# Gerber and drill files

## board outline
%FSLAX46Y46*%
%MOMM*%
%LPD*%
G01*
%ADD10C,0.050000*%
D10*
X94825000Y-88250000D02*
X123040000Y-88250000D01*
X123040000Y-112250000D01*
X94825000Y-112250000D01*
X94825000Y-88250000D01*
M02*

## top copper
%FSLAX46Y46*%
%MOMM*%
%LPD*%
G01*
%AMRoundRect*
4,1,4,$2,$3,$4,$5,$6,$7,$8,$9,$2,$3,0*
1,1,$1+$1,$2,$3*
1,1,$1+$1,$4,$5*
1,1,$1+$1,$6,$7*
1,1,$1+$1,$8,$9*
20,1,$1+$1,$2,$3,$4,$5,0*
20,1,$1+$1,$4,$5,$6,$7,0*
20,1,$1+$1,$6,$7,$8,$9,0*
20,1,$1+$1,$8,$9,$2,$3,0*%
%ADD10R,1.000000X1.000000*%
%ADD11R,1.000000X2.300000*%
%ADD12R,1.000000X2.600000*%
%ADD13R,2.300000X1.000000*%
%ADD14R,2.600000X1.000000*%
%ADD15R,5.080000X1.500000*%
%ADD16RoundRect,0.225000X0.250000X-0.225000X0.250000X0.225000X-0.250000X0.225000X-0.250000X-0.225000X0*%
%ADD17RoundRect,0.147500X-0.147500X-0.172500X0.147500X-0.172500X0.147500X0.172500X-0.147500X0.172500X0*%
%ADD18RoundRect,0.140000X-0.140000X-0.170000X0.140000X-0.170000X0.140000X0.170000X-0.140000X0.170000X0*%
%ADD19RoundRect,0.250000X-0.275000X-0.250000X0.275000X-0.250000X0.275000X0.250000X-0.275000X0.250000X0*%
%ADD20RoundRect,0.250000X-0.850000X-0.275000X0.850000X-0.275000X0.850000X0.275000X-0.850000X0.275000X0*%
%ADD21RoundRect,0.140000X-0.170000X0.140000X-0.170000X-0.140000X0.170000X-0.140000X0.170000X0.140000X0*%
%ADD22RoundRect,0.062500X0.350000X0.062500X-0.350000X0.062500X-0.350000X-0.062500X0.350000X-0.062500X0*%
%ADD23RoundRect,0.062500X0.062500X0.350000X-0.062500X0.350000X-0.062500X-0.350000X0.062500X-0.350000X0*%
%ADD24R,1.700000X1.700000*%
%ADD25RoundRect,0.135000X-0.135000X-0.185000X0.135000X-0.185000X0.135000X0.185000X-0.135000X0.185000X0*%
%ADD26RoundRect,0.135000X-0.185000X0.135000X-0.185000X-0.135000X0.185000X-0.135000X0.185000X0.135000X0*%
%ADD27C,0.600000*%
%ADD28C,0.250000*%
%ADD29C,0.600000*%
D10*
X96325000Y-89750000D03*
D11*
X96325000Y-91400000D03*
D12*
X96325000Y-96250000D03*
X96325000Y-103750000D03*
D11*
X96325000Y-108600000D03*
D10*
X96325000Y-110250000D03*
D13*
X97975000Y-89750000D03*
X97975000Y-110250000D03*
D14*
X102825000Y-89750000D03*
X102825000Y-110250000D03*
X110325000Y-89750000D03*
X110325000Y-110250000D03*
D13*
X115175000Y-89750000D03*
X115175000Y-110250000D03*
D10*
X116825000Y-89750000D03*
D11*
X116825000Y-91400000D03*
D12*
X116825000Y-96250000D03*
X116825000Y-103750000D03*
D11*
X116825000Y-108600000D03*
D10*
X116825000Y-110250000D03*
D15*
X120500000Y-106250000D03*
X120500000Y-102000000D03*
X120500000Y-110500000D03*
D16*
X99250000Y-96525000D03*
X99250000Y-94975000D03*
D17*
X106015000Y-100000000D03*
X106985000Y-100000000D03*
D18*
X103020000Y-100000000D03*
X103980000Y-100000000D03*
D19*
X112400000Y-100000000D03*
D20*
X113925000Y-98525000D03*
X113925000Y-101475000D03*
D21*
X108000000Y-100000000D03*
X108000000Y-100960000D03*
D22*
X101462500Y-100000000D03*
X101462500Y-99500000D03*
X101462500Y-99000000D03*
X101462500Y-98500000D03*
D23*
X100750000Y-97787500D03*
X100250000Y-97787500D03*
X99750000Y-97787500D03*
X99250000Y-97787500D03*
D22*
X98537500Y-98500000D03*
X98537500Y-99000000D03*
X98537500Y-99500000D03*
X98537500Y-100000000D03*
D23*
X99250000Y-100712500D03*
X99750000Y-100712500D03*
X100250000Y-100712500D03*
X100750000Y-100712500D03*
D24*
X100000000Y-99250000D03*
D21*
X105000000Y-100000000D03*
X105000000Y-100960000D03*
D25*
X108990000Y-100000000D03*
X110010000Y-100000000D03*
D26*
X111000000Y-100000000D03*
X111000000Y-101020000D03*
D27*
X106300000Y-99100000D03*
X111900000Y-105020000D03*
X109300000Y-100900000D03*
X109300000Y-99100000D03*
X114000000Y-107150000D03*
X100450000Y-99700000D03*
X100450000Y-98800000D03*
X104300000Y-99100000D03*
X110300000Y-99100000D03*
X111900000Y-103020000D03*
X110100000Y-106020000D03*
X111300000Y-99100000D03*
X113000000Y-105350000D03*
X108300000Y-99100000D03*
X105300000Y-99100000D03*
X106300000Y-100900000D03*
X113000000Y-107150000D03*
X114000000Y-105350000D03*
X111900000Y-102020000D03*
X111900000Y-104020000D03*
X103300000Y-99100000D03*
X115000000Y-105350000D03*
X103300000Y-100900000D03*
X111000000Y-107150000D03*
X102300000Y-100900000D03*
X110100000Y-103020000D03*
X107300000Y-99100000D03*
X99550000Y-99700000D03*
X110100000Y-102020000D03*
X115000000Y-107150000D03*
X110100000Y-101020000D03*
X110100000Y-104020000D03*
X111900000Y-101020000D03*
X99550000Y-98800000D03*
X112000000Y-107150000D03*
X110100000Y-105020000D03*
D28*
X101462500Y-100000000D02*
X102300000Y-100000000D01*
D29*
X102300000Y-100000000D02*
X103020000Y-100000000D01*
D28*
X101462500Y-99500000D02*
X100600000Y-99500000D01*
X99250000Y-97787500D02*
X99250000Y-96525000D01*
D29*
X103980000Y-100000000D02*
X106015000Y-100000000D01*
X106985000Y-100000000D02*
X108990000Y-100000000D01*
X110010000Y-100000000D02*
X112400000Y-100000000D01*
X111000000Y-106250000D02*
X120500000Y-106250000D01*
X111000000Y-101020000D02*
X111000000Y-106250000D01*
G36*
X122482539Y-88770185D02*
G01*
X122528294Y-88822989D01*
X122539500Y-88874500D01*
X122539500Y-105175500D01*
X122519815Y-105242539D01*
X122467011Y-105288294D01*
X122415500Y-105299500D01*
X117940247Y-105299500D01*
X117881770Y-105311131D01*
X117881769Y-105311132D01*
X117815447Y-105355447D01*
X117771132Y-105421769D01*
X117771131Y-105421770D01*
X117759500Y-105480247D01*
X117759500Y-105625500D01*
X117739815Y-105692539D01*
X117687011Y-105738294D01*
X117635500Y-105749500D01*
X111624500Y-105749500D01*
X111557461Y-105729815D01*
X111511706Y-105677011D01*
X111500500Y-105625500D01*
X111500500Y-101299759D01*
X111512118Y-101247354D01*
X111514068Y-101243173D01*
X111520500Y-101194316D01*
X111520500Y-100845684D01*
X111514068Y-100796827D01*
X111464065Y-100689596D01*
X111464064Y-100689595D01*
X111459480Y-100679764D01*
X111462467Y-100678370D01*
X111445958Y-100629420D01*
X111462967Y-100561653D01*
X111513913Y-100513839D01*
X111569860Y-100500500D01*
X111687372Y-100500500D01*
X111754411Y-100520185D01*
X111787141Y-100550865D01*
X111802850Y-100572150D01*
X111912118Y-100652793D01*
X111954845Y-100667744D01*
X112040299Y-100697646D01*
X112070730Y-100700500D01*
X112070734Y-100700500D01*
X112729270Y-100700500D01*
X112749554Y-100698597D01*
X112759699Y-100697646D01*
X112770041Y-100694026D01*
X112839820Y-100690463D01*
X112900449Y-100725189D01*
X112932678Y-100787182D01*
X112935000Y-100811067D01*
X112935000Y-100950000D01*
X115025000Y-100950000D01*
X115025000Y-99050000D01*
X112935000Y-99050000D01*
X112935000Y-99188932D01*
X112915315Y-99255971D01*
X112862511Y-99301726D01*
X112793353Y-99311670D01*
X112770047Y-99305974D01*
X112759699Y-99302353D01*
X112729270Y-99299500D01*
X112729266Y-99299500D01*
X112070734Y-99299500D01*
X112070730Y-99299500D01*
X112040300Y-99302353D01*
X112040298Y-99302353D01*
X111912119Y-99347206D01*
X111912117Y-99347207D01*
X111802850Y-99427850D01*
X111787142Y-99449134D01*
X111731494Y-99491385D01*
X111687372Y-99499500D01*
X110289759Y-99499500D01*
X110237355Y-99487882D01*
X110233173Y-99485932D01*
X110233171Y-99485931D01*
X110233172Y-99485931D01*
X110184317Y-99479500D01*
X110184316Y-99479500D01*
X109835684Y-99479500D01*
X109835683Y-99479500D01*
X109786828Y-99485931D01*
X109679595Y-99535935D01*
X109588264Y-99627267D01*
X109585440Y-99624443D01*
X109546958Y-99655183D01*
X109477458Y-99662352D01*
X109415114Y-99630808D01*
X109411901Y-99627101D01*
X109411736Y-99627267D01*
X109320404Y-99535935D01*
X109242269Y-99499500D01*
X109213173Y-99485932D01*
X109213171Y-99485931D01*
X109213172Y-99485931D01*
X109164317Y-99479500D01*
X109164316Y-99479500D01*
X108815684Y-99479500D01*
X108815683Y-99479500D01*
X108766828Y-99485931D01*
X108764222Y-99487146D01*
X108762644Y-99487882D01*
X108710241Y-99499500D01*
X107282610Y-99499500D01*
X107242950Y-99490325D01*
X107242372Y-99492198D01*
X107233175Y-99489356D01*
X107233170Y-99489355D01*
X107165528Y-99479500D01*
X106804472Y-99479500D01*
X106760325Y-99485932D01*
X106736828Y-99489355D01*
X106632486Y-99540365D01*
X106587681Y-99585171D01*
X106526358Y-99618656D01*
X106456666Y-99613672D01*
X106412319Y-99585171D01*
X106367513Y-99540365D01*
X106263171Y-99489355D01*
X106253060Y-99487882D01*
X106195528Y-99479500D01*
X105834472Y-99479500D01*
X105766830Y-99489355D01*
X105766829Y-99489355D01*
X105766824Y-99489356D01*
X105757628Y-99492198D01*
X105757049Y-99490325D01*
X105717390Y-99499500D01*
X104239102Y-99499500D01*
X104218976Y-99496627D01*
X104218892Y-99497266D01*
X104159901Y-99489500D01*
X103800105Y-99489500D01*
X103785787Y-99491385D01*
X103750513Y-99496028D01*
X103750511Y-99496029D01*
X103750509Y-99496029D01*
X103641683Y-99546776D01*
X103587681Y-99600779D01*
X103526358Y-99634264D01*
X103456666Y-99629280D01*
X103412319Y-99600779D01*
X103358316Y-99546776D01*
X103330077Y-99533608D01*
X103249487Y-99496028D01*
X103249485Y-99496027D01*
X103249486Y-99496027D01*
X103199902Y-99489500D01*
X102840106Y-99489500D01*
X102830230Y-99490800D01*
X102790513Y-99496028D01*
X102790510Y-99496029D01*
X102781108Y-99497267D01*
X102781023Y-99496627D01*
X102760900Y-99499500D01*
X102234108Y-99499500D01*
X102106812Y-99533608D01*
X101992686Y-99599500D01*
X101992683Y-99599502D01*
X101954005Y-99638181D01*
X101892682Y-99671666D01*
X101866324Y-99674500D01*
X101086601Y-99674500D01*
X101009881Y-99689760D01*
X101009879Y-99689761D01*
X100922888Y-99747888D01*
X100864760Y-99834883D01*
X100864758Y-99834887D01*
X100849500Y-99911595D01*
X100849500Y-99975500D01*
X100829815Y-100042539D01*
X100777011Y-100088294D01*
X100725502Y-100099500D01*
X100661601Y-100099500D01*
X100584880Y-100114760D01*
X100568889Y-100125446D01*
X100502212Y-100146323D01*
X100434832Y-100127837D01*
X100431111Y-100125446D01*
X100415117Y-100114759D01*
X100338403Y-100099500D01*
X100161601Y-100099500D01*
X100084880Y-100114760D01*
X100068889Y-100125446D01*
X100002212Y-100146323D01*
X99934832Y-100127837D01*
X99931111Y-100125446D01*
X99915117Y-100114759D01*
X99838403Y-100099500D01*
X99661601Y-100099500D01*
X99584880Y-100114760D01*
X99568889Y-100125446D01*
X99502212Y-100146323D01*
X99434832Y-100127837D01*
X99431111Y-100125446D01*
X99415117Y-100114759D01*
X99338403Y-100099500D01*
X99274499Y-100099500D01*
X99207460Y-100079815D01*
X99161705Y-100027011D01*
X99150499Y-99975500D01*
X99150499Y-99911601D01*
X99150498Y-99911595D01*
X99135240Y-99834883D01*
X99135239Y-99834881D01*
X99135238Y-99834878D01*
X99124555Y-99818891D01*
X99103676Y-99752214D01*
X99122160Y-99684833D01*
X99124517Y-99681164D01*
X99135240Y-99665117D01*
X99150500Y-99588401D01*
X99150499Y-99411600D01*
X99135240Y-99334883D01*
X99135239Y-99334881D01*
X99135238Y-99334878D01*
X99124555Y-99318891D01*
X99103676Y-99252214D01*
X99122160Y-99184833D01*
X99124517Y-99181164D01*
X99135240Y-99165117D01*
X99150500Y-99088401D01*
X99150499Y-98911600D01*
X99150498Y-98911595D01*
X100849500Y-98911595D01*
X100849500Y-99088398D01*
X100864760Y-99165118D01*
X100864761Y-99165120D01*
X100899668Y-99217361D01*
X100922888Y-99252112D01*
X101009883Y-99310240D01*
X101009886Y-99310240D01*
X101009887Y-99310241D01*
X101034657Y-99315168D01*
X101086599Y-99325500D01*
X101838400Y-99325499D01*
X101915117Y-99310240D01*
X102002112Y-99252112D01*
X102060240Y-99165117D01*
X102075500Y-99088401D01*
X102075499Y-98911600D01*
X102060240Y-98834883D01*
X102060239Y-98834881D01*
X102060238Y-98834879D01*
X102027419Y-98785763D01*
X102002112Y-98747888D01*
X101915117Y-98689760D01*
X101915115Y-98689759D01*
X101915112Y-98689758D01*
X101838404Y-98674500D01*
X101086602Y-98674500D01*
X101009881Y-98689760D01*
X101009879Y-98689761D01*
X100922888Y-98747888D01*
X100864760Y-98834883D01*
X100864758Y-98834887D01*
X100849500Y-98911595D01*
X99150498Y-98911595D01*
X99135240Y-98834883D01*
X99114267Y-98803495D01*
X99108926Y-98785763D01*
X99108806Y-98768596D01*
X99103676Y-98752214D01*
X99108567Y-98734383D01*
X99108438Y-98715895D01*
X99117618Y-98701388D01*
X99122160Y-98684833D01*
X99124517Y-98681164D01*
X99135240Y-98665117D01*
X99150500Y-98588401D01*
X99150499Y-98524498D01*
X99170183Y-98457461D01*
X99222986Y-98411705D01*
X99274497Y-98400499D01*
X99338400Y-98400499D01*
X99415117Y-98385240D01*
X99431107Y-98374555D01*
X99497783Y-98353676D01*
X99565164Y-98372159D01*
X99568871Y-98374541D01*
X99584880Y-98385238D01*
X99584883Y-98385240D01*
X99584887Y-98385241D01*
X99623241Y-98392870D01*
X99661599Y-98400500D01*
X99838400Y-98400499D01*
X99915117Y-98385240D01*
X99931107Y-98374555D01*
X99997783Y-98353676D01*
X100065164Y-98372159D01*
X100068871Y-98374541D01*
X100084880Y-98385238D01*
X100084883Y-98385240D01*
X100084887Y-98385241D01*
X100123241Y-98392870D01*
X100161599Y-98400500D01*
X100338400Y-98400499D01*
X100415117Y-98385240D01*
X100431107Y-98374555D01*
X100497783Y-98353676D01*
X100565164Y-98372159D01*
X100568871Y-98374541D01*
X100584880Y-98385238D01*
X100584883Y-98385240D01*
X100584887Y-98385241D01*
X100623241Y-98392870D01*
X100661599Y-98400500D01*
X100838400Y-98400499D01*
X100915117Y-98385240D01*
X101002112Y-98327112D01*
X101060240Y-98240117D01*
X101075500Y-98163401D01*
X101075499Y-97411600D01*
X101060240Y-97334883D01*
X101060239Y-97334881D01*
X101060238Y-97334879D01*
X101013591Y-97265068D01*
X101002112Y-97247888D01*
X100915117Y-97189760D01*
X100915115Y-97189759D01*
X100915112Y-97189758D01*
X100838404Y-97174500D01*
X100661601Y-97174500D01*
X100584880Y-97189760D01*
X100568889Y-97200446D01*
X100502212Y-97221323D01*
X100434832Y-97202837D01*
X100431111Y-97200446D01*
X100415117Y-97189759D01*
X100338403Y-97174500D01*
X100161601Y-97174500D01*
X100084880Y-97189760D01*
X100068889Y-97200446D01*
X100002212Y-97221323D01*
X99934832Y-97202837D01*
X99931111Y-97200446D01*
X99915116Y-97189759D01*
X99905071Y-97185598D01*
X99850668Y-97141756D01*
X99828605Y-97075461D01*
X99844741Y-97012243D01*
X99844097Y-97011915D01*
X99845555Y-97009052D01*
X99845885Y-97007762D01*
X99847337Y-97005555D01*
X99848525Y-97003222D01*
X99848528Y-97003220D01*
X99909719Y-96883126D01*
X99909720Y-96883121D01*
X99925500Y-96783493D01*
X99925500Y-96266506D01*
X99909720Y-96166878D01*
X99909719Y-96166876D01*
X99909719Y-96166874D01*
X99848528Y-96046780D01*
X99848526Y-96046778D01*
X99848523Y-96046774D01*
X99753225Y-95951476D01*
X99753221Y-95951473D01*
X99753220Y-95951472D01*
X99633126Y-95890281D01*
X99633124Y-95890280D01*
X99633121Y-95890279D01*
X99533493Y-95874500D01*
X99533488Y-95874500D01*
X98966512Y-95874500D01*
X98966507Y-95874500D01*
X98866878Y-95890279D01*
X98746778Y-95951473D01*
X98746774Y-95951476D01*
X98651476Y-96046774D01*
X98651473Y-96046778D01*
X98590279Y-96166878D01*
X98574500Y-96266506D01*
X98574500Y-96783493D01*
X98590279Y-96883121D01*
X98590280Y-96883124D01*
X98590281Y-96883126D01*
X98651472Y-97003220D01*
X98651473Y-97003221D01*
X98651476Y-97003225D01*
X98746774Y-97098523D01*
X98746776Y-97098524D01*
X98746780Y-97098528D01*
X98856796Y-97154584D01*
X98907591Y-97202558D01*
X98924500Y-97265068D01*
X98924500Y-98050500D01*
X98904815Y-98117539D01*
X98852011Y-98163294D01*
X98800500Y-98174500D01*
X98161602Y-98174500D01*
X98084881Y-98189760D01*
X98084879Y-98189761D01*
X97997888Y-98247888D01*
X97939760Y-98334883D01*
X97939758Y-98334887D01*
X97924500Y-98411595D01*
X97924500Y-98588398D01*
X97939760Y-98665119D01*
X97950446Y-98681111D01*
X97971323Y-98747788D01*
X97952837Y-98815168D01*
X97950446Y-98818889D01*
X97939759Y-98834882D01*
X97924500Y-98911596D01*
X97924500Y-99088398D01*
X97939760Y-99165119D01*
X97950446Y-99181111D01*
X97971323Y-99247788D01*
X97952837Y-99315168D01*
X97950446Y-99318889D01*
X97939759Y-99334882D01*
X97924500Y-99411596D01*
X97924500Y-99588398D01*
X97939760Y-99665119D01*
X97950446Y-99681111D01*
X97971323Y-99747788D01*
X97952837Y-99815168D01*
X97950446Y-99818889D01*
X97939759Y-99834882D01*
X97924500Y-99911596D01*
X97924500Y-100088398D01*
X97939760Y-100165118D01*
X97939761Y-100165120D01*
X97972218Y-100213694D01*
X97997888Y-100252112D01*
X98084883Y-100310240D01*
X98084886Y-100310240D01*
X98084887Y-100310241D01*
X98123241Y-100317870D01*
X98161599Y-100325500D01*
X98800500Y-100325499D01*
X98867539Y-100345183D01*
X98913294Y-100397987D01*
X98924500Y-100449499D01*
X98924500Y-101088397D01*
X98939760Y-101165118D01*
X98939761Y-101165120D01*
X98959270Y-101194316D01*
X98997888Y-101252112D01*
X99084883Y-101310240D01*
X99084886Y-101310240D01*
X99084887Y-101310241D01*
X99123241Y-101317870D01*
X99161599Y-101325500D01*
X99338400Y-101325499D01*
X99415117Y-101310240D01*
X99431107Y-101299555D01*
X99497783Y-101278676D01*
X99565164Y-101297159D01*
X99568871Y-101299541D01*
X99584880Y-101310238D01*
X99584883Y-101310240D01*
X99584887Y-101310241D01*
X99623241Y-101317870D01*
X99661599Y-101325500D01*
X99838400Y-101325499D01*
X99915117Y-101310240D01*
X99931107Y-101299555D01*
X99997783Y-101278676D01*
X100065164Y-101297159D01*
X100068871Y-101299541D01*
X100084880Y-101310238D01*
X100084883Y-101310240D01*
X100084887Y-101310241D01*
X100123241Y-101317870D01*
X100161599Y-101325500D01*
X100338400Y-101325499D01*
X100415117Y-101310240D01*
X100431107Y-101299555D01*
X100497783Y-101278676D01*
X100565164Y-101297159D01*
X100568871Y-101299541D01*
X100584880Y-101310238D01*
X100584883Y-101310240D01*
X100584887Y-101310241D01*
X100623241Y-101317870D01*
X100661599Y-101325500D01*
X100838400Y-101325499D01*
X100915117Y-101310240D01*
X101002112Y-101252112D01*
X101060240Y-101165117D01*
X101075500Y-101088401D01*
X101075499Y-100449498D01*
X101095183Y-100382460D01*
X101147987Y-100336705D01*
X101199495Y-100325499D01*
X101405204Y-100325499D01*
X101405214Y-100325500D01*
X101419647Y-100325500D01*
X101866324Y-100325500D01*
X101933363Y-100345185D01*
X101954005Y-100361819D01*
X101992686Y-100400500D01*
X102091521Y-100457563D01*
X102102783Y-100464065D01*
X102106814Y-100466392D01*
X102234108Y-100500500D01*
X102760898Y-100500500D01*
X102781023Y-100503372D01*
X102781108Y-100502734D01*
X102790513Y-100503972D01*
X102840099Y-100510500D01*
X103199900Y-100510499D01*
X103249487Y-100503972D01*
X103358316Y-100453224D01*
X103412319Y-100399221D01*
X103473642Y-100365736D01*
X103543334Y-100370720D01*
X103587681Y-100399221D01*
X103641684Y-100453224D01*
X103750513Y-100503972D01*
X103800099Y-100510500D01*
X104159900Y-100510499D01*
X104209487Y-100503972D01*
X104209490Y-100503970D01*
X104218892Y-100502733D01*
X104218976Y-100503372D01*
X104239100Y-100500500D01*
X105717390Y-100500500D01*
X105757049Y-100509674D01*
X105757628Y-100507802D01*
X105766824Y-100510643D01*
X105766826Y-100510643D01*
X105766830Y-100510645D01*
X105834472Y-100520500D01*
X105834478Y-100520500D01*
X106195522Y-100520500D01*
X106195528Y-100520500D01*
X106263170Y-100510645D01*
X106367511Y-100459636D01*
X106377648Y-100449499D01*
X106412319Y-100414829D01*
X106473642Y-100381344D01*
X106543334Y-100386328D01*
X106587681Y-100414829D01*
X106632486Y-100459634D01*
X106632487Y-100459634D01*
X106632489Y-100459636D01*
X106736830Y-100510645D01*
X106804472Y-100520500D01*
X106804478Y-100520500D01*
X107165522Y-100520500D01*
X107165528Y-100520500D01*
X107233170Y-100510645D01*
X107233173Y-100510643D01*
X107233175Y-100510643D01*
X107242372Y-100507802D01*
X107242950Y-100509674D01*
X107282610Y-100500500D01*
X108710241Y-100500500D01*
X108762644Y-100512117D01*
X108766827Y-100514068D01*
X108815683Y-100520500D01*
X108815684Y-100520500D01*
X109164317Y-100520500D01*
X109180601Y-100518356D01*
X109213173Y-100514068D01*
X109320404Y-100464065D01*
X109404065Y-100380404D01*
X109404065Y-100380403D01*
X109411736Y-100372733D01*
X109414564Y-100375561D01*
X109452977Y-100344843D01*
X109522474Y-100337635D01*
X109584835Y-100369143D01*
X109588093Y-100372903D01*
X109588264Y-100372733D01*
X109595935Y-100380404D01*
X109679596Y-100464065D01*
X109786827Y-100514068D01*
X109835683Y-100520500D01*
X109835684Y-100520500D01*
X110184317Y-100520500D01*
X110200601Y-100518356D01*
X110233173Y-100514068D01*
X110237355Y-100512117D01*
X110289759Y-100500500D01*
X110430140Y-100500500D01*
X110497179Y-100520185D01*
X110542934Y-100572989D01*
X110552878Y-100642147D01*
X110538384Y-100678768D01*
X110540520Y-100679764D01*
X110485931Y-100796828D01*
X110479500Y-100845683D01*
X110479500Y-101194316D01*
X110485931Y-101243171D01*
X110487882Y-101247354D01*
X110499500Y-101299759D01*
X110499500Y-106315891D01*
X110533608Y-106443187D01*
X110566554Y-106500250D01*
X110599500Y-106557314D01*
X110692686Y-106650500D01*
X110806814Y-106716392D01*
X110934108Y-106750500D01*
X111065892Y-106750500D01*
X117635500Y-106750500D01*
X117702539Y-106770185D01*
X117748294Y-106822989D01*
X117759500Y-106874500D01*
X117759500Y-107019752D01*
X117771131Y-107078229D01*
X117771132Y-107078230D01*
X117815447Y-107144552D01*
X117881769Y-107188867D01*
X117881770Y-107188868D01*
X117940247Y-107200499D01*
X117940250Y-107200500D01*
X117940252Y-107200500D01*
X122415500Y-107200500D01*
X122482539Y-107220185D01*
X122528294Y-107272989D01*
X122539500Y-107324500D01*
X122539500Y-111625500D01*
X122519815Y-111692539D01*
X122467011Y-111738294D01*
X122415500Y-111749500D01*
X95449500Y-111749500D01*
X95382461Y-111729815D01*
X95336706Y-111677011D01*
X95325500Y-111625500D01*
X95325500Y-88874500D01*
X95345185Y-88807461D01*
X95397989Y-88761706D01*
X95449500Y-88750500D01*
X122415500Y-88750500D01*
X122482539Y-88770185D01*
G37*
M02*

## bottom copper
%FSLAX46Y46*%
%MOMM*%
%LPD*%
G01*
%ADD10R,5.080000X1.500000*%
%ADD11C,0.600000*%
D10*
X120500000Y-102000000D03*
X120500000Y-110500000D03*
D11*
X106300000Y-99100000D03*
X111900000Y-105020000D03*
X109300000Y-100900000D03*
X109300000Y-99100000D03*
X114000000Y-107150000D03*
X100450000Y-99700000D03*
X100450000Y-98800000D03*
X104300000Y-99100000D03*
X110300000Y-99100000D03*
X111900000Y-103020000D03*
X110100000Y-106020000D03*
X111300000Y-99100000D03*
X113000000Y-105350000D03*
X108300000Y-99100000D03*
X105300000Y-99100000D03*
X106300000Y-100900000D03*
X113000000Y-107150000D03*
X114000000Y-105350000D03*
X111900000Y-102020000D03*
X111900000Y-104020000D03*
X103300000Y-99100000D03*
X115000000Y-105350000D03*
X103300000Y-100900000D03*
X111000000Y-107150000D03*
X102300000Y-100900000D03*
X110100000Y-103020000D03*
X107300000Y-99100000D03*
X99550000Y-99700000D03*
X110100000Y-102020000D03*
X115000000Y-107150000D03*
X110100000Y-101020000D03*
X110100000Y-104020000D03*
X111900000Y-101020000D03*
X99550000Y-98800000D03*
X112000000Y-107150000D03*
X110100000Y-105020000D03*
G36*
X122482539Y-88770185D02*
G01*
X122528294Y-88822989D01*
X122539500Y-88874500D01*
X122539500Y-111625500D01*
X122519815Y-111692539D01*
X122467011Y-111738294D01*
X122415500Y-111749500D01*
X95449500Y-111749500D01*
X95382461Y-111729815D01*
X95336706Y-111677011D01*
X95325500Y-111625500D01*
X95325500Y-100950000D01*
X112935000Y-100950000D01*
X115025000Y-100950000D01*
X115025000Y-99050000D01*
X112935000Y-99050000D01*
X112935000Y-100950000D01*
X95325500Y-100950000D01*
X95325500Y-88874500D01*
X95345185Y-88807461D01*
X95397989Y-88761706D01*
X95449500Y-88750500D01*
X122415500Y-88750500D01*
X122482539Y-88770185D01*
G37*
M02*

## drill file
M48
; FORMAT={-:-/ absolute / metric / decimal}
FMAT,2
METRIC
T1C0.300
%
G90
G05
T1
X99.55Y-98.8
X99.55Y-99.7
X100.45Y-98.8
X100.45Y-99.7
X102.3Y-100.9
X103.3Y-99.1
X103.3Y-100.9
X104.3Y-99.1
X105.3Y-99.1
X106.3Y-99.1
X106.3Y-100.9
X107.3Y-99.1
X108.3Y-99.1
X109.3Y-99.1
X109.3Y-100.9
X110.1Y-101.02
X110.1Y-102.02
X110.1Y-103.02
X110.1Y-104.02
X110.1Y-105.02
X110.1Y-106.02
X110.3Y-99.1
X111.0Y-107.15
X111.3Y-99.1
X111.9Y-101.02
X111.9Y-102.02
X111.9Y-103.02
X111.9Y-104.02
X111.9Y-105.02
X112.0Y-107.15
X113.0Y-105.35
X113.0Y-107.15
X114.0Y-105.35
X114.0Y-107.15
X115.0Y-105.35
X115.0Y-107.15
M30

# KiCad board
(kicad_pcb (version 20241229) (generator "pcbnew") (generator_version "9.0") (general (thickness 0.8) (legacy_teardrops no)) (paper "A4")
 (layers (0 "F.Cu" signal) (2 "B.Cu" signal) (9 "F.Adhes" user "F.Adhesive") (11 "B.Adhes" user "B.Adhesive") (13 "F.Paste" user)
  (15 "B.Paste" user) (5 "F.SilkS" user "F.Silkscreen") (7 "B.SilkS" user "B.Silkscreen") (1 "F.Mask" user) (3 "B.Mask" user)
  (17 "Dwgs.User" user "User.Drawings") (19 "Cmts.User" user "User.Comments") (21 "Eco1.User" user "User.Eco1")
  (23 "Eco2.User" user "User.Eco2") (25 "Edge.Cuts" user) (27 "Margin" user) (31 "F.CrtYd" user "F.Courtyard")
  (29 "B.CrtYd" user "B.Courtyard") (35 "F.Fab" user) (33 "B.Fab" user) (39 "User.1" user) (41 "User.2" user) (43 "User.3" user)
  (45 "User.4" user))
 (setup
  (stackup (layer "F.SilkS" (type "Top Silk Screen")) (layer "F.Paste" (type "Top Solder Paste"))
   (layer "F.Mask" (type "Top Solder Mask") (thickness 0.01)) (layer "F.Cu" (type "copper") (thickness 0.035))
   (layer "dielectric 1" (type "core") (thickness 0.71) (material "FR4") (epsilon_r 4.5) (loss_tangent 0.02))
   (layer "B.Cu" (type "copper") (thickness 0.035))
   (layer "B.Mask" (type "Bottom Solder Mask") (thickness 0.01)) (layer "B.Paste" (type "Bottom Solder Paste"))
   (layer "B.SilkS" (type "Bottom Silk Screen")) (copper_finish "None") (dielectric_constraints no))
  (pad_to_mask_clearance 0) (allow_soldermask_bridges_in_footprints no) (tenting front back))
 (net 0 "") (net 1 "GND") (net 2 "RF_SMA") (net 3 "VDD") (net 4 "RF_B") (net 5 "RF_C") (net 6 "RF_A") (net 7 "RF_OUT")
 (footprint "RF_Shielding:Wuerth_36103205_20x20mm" (layer "F.Cu") (at 106.575 100)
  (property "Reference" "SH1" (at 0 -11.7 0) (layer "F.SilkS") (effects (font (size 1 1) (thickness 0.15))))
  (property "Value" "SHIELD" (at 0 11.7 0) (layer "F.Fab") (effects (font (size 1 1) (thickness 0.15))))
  (pad "1" smd rect (at -10.25 -10.25) (size 1 1) (layers "F.Cu" "F.Mask" "F.Paste") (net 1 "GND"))
  (pad "1" smd rect (at -10.25 -8.6) (size 1 2.3) (layers "F.Cu" "F.Mask" "F.Paste") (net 1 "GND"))
  (pad "1" smd rect (at -10.25 -3.75) (size 1 2.6) (layers "F.Cu" "F.Mask" "F.Paste") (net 1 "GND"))
  (pad "1" smd rect (at -10.25 3.75) (size 1 2.6) (layers "F.Cu" "F.Mask" "F.Paste") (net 1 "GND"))
  (pad "1" smd rect (at -10.25 8.6) (size 1 2.3) (layers "F.Cu" "F.Mask" "F.Paste") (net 1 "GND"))
  (pad "1" smd rect (at -10.25 10.25) (size 1 1) (layers "F.Cu" "F.Mask" "F.Paste") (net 1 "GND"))
  (pad "1" smd rect (at -8.6 -10.25) (size 2.3 1) (layers "F.Cu" "F.Mask" "F.Paste") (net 1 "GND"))
  (pad "1" smd rect (at -8.6 10.25) (size 2.3 1) (layers "F.Cu" "F.Mask" "F.Paste") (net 1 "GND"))
  (pad "1" smd rect (at -3.75 -10.25) (size 2.6 1) (layers "F.Cu" "F.Mask" "F.Paste") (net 1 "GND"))
  (pad "1" smd rect (at -3.75 10.25) (size 2.6 1) (layers "F.Cu" "F.Mask" "F.Paste") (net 1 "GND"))
  (pad "1" smd rect (at 3.75 -10.25) (size 2.6 1) (layers "F.Cu" "F.Mask" "F.Paste") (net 1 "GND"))
  (pad "1" smd rect (at 3.75 10.25) (size 2.6 1) (layers "F.Cu" "F.Mask" "F.Paste") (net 1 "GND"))
  (pad "1" smd rect (at 8.6 -10.25) (size 2.3 1) (layers "F.Cu" "F.Mask" "F.Paste") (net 1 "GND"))
  (pad "1" smd rect (at 8.6 10.25) (size 2.3 1) (layers "F.Cu" "F.Mask" "F.Paste") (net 1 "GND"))
  (pad "1" smd rect (at 10.25 -10.25) (size 1 1) (layers "F.Cu" "F.Mask" "F.Paste") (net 1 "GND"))
  (pad "1" smd rect (at 10.25 -8.6) (size 1 2.3) (layers "F.Cu" "F.Mask" "F.Paste") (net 1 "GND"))
  (pad "1" smd rect (at 10.25 -3.75) (size 1 2.6) (layers "F.Cu" "F.Mask" "F.Paste") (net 1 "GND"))
  (pad "1" smd rect (at 10.25 3.75) (size 1 2.6) (layers "F.Cu" "F.Mask" "F.Paste") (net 1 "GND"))
  (pad "1" smd rect (at 10.25 8.6) (size 1 2.3) (layers "F.Cu" "F.Mask" "F.Paste") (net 1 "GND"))
  (pad "1" smd rect (at 10.25 10.25) (size 1 1) (layers "F.Cu" "F.Mask" "F.Paste") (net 1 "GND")))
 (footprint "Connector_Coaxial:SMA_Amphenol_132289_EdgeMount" (layer "F.Cu") (at 120.5 106.25)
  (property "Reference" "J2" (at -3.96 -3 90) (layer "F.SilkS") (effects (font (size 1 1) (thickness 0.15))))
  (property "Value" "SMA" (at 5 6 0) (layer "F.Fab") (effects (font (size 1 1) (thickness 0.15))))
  (pad "1" smd rect (at 0 0 90) (size 1.5 5.08) (layers "F.Cu" "F.Mask" "F.Paste") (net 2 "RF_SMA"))
  (pad "2" smd rect (at 0 -4.25 90) (size 1.5 5.08) (layers "F.Cu" "F.Mask" "F.Paste") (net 1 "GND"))
  (pad "2" smd rect (at 0 -4.25 90) (size 1.5 5.08) (layers "B.Cu" "B.Mask" "B.Paste") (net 1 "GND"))
  (pad "2" smd rect (at 0 4.25 90) (size 1.5 5.08) (layers "F.Cu" "F.Mask" "F.Paste") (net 1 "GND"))
  (pad "2" smd rect (at 0 4.25 90) (size 1.5 5.08) (layers "B.Cu" "B.Mask" "B.Paste") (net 1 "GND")))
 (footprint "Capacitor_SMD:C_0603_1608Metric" (layer "F.Cu") (at 99.25 95.75 90)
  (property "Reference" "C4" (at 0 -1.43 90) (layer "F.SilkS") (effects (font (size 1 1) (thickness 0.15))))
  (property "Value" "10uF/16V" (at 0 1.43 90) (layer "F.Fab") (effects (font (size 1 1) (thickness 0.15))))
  (pad "1" smd roundrect (at -0.775 0 90) (size 0.9 0.95) (layers "F.Cu" "F.Mask" "F.Paste") (roundrect_rratio 0.25) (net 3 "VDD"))
  (pad "2" smd roundrect (at 0.775 0 90) (size 0.9 0.95) (layers "F.Cu" "F.Mask" "F.Paste") (roundrect_rratio 0.25) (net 1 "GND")))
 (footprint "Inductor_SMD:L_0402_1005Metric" (layer "F.Cu") (at 106.5 100)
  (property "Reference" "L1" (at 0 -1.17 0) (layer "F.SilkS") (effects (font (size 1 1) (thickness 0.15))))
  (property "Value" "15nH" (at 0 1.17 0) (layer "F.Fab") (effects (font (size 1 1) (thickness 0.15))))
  (pad "1" smd roundrect (at -0.485 0) (size 0.59 0.64) (layers "F.Cu" "F.Mask" "F.Paste") (roundrect_rratio 0.25) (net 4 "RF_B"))
  (pad "2" smd roundrect (at 0.485 0) (size 0.59 0.64) (layers "F.Cu" "F.Mask" "F.Paste") (roundrect_rratio 0.25) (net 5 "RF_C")))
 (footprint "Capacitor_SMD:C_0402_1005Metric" (layer "F.Cu") (at 103.5 100)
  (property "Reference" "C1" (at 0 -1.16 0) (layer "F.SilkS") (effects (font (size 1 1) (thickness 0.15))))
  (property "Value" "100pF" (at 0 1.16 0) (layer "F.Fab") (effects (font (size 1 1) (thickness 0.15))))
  (pad "1" smd roundrect (at -0.48 0) (size 0.56 0.62) (layers "F.Cu" "F.Mask" "F.Paste") (roundrect_rratio 0.25) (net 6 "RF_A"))
  (pad "2" smd roundrect (at 0.48 0) (size 0.56 0.62) (layers "F.Cu" "F.Mask" "F.Paste") (roundrect_rratio 0.25) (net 4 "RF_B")))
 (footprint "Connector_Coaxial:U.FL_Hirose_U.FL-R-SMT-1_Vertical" (layer "F.Cu") (at 113.45 100)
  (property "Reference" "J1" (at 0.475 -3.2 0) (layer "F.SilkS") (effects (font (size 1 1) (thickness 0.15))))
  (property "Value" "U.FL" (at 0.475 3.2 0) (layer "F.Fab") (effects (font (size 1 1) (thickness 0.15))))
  (pad "1" smd roundrect (at -1.05 0) (size 1.05 1) (layers "F.Cu" "F.Mask" "F.Paste") (roundrect_rratio 0.25) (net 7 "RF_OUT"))
  (pad "2" smd roundrect (at 0.475 -1.475) (size 2.2 1.05) (layers "F.Cu" "F.Mask" "F.Paste") (roundrect_rratio 0.2380952381) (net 1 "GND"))
  (pad "2" smd roundrect (at 0.475 1.475) (size 2.2 1.05) (layers "F.Cu" "F.Mask" "F.Paste") (roundrect_rratio 0.2380952381) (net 1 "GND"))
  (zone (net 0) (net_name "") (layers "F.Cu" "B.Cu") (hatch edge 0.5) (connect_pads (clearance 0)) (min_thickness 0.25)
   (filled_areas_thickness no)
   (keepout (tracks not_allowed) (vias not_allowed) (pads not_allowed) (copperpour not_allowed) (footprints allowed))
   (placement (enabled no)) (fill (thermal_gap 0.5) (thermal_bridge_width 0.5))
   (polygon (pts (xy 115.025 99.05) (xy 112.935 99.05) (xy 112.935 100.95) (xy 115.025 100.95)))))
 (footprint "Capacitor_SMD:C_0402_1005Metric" (layer "F.Cu") (at 108 100.48 -90)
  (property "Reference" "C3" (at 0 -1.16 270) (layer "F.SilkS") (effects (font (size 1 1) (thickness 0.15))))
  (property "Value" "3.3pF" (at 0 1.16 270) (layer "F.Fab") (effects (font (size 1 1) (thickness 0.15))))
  (pad "1" smd roundrect (at -0.48 0 270) (size 0.56 0.62) (layers "F.Cu" "F.Mask" "F.Paste") (roundrect_rratio 0.25) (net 5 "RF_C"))
  (pad "2" smd roundrect (at 0.48 0 270) (size 0.56 0.62) (layers "F.Cu" "F.Mask" "F.Paste") (roundrect_rratio 0.25) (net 1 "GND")))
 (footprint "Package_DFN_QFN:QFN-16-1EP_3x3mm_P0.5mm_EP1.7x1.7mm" (layer "F.Cu") (at 100 99.25 180)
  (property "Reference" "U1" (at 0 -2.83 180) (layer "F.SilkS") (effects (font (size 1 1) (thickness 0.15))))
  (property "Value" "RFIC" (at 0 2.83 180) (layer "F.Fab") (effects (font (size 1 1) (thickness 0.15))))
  (pad "" smd roundrect (at -0.425 -0.425 180) (size 0.69 0.69) (layers "F.Paste") (roundrect_rratio 0.25))
  (pad "" smd roundrect (at -0.425 0.425 180) (size 0.69 0.69) (layers "F.Paste") (roundrect_rratio 0.25))
  (pad "" smd roundrect (at 0.425 -0.425 180) (size 0.69 0.69) (layers "F.Paste") (roundrect_rratio 0.25))
  (pad "" smd roundrect (at 0.425 0.425 180) (size 0.69 0.69) (layers "F.Paste") (roundrect_rratio 0.25))
  (pad "1" smd roundrect (at -1.4625 -0.75 180) (size 0.825 0.25) (layers "F.Cu" "F.Mask" "F.Paste") (roundrect_rratio 0.25) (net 6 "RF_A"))
  (pad "2" smd roundrect (at -1.4625 -0.25 180) (size 0.825 0.25) (layers "F.Cu" "F.Mask" "F.Paste") (roundrect_rratio 0.25) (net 1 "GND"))
  (pad "3" smd roundrect (at -1.4625 0.25 180) (size 0.825 0.25) (layers "F.Cu" "F.Mask" "F.Paste") (roundrect_rratio 0.25))
  (pad "4" smd roundrect (at -1.4625 0.75 180) (size 0.825 0.25) (layers "F.Cu" "F.Mask" "F.Paste") (roundrect_rratio 0.25) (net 1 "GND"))
  (pad "5" smd roundrect (at -0.75 1.4625 180) (size 0.25 0.825) (layers "F.Cu" "F.Mask" "F.Paste") (roundrect_rratio 0.25))
  (pad "6" smd roundrect (at -0.25 1.4625 180) (size 0.25 0.825) (layers "F.Cu" "F.Mask" "F.Paste") (roundrect_rratio 0.25))
  (pad "7" smd roundrect (at 0.25 1.4625 180) (size 0.25 0.825) (layers "F.Cu" "F.Mask" "F.Paste") (roundrect_rratio 0.25))
  (pad "8" smd roundrect (at 0.75 1.4625 180) (size 0.25 0.825) (layers "F.Cu" "F.Mask" "F.Paste") (roundrect_rratio 0.25) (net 3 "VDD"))
  (pad "9" smd roundrect (at 1.4625 0.75 180) (size 0.825 0.25) (layers "F.Cu" "F.Mask" "F.Paste") (roundrect_rratio 0.25))
  (pad "10" smd roundrect (at 1.4625 0.25 180) (size 0.825 0.25) (layers "F.Cu" "F.Mask" "F.Paste") (roundrect_rratio 0.25))
  (pad "11" smd roundrect (at 1.4625 -0.25 180) (size 0.825 0.25) (layers "F.Cu" "F.Mask" "F.Paste") (roundrect_rratio 0.25))
  (pad "12" smd roundrect (at 1.4625 -0.75 180) (size 0.825 0.25) (layers "F.Cu" "F.Mask" "F.Paste") (roundrect_rratio 0.25))
  (pad "13" smd roundrect (at 0.75 -1.4625 180) (size 0.25 0.825) (layers "F.Cu" "F.Mask" "F.Paste") (roundrect_rratio 0.25))
  (pad "14" smd roundrect (at 0.25 -1.4625 180) (size 0.25 0.825) (layers "F.Cu" "F.Mask" "F.Paste") (roundrect_rratio 0.25))
  (pad "15" smd roundrect (at -0.25 -1.4625 180) (size 0.25 0.825) (layers "F.Cu" "F.Mask" "F.Paste") (roundrect_rratio 0.25))
  (pad "16" smd roundrect (at -0.75 -1.4625 180) (size 0.25 0.825) (layers "F.Cu" "F.Mask" "F.Paste") (roundrect_rratio 0.25))
  (pad "17" smd rect (at 0 0 180) (size 1.7 1.7) (layers "F.Cu" "F.Mask") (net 1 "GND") (zone_connect 2)))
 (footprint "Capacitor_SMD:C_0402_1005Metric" (layer "F.Cu") (at 105 100.48 -90)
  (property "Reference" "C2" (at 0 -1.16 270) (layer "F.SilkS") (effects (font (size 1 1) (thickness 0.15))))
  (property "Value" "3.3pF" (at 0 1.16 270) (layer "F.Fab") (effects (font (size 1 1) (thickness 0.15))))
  (pad "1" smd roundrect (at -0.48 0 270) (size 0.56 0.62) (layers "F.Cu" "F.Mask" "F.Paste") (roundrect_rratio 0.25) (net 4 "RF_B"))
  (pad "2" smd roundrect (at 0.48 0 270) (size 0.56 0.62) (layers "F.Cu" "F.Mask" "F.Paste") (roundrect_rratio 0.25) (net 1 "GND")))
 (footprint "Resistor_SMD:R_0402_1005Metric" (layer "F.Cu") (at 109.5 100)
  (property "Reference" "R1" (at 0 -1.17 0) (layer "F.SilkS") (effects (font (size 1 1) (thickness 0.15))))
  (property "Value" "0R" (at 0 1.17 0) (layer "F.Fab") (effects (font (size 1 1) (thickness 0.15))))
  (pad "1" smd roundrect (at -0.51 0) (size 0.54 0.64) (layers "F.Cu" "F.Mask" "F.Paste") (roundrect_rratio 0.25) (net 5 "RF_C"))
  (pad "2" smd roundrect (at 0.51 0) (size 0.54 0.64) (layers "F.Cu" "F.Mask" "F.Paste") (roundrect_rratio 0.25) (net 7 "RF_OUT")))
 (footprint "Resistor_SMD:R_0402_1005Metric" (layer "F.Cu") (at 111 100.51 -90)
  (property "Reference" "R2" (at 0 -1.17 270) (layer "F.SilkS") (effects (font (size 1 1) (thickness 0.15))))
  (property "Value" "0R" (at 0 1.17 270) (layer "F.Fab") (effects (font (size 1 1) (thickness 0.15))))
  (pad "1" smd roundrect (at -0.51 0 270) (size 0.54 0.64) (layers "F.Cu" "F.Mask" "F.Paste") (roundrect_rratio 0.25) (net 7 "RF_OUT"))
  (pad "2" smd roundrect (at 0.51 0 270) (size 0.54 0.64) (layers "F.Cu" "F.Mask" "F.Paste") (roundrect_rratio 0.25) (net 2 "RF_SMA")))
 (gr_rect (start 94.825 88.25) (end 123.04 112.25) (stroke (width 0.05) (type default)) (fill no) (layer "Edge.Cuts"))
 (segment (start 101.4625 100) (end 102.3 100) (width 0.25) (layer "F.Cu") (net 6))
 (segment (start 102.3 100) (end 103.02 100) (width 0.6) (layer "F.Cu") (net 6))
 (segment (start 101.4625 99.5) (end 100.6 99.5) (width 0.25) (layer "F.Cu") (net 1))
 (via (at 106.3 99.1) (size 0.6) (drill 0.3) (layers "F.Cu" "B.Cu") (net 1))
 (via (at 111.9 105.02) (size 0.6) (drill 0.3) (layers "F.Cu" "B.Cu") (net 1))
 (via (at 109.3 100.9) (size 0.6) (drill 0.3) (layers "F.Cu" "B.Cu") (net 1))
 (via (at 109.3 99.1) (size 0.6) (drill 0.3) (layers "F.Cu" "B.Cu") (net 1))
 (via (at 114 107.15) (size 0.6) (drill 0.3) (layers "F.Cu" "B.Cu") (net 1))
 (via (at 100.45 99.7) (size 0.6) (drill 0.3) (layers "F.Cu" "B.Cu") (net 1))
 (via (at 100.45 98.8) (size 0.6) (drill 0.3) (layers "F.Cu" "B.Cu") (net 1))
 (via (at 104.3 99.1) (size 0.6) (drill 0.3) (layers "F.Cu" "B.Cu") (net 1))
 (via (at 110.3 99.1) (size 0.6) (drill 0.3) (layers "F.Cu" "B.Cu") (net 1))
 (via (at 111.9 103.02) (size 0.6) (drill 0.3) (layers "F.Cu" "B.Cu") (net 1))
 (via (at 110.1 106.02) (size 0.6) (drill 0.3) (layers "F.Cu" "B.Cu") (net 1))
 (via (at 111.3 99.1) (size 0.6) (drill 0.3) (layers "F.Cu" "B.Cu") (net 1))
 (via (at 113 105.35) (size 0.6) (drill 0.3) (layers "F.Cu" "B.Cu") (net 1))
 (via (at 108.3 99.1) (size 0.6) (drill 0.3) (layers "F.Cu" "B.Cu") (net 1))
 (via (at 105.3 99.1) (size 0.6) (drill 0.3) (layers "F.Cu" "B.Cu") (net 1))
 (via (at 106.3 100.9) (size 0.6) (drill 0.3) (layers "F.Cu" "B.Cu") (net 1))
 (via (at 113 107.15) (size 0.6) (drill 0.3) (layers "F.Cu" "B.Cu") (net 1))
 (via (at 114 105.35) (size 0.6) (drill 0.3) (layers "F.Cu" "B.Cu") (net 1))
 (via (at 111.9 102.02) (size 0.6) (drill 0.3) (layers "F.Cu" "B.Cu") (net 1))
 (via (at 111.9 104.02) (size 0.6) (drill 0.3) (layers "F.Cu" "B.Cu") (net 1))
 (via (at 103.3 99.1) (size 0.6) (drill 0.3) (layers "F.Cu" "B.Cu") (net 1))
 (via (at 115 105.35) (size 0.6) (drill 0.3) (layers "F.Cu" "B.Cu") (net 1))
 (via (at 103.3 100.9) (size 0.6) (drill 0.3) (layers "F.Cu" "B.Cu") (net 1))
 (via (at 111 107.15) (size 0.6) (drill 0.3) (layers "F.Cu" "B.Cu") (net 1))
 (via (at 102.3 100.9) (size 0.6) (drill 0.3) (layers "F.Cu" "B.Cu") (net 1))
 (via (at 110.1 103.02) (size 0.6) (drill 0.3) (layers "F.Cu" "B.Cu") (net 1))
 (via (at 107.3 99.1) (size 0.6) (drill 0.3) (layers "F.Cu" "B.Cu") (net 1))
 (via (at 99.55 99.7) (size 0.6) (drill 0.3) (layers "F.Cu" "B.Cu") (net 1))
 (via (at 110.1 102.02) (size 0.6) (drill 0.3) (layers "F.Cu" "B.Cu") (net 1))
 (via (at 115 107.15) (size 0.6) (drill 0.3) (layers "F.Cu" "B.Cu") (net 1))
 (via (at 110.1 101.02) (size 0.6) (drill 0.3) (layers "F.Cu" "B.Cu") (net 1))
 (via (at 110.1 104.02) (size 0.6) (drill 0.3) (layers "F.Cu" "B.Cu") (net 1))
 (via (at 111.9 101.02) (size 0.6) (drill 0.3) (layers "F.Cu" "B.Cu") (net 1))
 (via (at 99.55 98.8) (size 0.6) (drill 0.3) (layers "F.Cu" "B.Cu") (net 1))
 (via (at 112 107.15) (size 0.6) (drill 0.3) (layers "F.Cu" "B.Cu") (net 1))
 (via (at 110.1 105.02) (size 0.6) (drill 0.3) (layers "F.Cu" "B.Cu") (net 1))
 (segment (start 99.25 97.7875) (end 99.25 96.525) (width 0.25) (layer "F.Cu") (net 3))
 (segment (start 103.98 100) (end 106.015 100) (width 0.6) (layer "F.Cu") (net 4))
 (segment (start 106.985 100) (end 108.99 100) (width 0.6) (layer "F.Cu") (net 5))
 (segment (start 110.01 100) (end 112.4 100) (width 0.6) (layer "F.Cu") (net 7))
 (segment (start 111 106.25) (end 120.5 106.25) (width 0.6) (layer "F.Cu") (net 2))
 (segment (start 111 101.02) (end 111 106.25) (width 0.6) (layer "F.Cu") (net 2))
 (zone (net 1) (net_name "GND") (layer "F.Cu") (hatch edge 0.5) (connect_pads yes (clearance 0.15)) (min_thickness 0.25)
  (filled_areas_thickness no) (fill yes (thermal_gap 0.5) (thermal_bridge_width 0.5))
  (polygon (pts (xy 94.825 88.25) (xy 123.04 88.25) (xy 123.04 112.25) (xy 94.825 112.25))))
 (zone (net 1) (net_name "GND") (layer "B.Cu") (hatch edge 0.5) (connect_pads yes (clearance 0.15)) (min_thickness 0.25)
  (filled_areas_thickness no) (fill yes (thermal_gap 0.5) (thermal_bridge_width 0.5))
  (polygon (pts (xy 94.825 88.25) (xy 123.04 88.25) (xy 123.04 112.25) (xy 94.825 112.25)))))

